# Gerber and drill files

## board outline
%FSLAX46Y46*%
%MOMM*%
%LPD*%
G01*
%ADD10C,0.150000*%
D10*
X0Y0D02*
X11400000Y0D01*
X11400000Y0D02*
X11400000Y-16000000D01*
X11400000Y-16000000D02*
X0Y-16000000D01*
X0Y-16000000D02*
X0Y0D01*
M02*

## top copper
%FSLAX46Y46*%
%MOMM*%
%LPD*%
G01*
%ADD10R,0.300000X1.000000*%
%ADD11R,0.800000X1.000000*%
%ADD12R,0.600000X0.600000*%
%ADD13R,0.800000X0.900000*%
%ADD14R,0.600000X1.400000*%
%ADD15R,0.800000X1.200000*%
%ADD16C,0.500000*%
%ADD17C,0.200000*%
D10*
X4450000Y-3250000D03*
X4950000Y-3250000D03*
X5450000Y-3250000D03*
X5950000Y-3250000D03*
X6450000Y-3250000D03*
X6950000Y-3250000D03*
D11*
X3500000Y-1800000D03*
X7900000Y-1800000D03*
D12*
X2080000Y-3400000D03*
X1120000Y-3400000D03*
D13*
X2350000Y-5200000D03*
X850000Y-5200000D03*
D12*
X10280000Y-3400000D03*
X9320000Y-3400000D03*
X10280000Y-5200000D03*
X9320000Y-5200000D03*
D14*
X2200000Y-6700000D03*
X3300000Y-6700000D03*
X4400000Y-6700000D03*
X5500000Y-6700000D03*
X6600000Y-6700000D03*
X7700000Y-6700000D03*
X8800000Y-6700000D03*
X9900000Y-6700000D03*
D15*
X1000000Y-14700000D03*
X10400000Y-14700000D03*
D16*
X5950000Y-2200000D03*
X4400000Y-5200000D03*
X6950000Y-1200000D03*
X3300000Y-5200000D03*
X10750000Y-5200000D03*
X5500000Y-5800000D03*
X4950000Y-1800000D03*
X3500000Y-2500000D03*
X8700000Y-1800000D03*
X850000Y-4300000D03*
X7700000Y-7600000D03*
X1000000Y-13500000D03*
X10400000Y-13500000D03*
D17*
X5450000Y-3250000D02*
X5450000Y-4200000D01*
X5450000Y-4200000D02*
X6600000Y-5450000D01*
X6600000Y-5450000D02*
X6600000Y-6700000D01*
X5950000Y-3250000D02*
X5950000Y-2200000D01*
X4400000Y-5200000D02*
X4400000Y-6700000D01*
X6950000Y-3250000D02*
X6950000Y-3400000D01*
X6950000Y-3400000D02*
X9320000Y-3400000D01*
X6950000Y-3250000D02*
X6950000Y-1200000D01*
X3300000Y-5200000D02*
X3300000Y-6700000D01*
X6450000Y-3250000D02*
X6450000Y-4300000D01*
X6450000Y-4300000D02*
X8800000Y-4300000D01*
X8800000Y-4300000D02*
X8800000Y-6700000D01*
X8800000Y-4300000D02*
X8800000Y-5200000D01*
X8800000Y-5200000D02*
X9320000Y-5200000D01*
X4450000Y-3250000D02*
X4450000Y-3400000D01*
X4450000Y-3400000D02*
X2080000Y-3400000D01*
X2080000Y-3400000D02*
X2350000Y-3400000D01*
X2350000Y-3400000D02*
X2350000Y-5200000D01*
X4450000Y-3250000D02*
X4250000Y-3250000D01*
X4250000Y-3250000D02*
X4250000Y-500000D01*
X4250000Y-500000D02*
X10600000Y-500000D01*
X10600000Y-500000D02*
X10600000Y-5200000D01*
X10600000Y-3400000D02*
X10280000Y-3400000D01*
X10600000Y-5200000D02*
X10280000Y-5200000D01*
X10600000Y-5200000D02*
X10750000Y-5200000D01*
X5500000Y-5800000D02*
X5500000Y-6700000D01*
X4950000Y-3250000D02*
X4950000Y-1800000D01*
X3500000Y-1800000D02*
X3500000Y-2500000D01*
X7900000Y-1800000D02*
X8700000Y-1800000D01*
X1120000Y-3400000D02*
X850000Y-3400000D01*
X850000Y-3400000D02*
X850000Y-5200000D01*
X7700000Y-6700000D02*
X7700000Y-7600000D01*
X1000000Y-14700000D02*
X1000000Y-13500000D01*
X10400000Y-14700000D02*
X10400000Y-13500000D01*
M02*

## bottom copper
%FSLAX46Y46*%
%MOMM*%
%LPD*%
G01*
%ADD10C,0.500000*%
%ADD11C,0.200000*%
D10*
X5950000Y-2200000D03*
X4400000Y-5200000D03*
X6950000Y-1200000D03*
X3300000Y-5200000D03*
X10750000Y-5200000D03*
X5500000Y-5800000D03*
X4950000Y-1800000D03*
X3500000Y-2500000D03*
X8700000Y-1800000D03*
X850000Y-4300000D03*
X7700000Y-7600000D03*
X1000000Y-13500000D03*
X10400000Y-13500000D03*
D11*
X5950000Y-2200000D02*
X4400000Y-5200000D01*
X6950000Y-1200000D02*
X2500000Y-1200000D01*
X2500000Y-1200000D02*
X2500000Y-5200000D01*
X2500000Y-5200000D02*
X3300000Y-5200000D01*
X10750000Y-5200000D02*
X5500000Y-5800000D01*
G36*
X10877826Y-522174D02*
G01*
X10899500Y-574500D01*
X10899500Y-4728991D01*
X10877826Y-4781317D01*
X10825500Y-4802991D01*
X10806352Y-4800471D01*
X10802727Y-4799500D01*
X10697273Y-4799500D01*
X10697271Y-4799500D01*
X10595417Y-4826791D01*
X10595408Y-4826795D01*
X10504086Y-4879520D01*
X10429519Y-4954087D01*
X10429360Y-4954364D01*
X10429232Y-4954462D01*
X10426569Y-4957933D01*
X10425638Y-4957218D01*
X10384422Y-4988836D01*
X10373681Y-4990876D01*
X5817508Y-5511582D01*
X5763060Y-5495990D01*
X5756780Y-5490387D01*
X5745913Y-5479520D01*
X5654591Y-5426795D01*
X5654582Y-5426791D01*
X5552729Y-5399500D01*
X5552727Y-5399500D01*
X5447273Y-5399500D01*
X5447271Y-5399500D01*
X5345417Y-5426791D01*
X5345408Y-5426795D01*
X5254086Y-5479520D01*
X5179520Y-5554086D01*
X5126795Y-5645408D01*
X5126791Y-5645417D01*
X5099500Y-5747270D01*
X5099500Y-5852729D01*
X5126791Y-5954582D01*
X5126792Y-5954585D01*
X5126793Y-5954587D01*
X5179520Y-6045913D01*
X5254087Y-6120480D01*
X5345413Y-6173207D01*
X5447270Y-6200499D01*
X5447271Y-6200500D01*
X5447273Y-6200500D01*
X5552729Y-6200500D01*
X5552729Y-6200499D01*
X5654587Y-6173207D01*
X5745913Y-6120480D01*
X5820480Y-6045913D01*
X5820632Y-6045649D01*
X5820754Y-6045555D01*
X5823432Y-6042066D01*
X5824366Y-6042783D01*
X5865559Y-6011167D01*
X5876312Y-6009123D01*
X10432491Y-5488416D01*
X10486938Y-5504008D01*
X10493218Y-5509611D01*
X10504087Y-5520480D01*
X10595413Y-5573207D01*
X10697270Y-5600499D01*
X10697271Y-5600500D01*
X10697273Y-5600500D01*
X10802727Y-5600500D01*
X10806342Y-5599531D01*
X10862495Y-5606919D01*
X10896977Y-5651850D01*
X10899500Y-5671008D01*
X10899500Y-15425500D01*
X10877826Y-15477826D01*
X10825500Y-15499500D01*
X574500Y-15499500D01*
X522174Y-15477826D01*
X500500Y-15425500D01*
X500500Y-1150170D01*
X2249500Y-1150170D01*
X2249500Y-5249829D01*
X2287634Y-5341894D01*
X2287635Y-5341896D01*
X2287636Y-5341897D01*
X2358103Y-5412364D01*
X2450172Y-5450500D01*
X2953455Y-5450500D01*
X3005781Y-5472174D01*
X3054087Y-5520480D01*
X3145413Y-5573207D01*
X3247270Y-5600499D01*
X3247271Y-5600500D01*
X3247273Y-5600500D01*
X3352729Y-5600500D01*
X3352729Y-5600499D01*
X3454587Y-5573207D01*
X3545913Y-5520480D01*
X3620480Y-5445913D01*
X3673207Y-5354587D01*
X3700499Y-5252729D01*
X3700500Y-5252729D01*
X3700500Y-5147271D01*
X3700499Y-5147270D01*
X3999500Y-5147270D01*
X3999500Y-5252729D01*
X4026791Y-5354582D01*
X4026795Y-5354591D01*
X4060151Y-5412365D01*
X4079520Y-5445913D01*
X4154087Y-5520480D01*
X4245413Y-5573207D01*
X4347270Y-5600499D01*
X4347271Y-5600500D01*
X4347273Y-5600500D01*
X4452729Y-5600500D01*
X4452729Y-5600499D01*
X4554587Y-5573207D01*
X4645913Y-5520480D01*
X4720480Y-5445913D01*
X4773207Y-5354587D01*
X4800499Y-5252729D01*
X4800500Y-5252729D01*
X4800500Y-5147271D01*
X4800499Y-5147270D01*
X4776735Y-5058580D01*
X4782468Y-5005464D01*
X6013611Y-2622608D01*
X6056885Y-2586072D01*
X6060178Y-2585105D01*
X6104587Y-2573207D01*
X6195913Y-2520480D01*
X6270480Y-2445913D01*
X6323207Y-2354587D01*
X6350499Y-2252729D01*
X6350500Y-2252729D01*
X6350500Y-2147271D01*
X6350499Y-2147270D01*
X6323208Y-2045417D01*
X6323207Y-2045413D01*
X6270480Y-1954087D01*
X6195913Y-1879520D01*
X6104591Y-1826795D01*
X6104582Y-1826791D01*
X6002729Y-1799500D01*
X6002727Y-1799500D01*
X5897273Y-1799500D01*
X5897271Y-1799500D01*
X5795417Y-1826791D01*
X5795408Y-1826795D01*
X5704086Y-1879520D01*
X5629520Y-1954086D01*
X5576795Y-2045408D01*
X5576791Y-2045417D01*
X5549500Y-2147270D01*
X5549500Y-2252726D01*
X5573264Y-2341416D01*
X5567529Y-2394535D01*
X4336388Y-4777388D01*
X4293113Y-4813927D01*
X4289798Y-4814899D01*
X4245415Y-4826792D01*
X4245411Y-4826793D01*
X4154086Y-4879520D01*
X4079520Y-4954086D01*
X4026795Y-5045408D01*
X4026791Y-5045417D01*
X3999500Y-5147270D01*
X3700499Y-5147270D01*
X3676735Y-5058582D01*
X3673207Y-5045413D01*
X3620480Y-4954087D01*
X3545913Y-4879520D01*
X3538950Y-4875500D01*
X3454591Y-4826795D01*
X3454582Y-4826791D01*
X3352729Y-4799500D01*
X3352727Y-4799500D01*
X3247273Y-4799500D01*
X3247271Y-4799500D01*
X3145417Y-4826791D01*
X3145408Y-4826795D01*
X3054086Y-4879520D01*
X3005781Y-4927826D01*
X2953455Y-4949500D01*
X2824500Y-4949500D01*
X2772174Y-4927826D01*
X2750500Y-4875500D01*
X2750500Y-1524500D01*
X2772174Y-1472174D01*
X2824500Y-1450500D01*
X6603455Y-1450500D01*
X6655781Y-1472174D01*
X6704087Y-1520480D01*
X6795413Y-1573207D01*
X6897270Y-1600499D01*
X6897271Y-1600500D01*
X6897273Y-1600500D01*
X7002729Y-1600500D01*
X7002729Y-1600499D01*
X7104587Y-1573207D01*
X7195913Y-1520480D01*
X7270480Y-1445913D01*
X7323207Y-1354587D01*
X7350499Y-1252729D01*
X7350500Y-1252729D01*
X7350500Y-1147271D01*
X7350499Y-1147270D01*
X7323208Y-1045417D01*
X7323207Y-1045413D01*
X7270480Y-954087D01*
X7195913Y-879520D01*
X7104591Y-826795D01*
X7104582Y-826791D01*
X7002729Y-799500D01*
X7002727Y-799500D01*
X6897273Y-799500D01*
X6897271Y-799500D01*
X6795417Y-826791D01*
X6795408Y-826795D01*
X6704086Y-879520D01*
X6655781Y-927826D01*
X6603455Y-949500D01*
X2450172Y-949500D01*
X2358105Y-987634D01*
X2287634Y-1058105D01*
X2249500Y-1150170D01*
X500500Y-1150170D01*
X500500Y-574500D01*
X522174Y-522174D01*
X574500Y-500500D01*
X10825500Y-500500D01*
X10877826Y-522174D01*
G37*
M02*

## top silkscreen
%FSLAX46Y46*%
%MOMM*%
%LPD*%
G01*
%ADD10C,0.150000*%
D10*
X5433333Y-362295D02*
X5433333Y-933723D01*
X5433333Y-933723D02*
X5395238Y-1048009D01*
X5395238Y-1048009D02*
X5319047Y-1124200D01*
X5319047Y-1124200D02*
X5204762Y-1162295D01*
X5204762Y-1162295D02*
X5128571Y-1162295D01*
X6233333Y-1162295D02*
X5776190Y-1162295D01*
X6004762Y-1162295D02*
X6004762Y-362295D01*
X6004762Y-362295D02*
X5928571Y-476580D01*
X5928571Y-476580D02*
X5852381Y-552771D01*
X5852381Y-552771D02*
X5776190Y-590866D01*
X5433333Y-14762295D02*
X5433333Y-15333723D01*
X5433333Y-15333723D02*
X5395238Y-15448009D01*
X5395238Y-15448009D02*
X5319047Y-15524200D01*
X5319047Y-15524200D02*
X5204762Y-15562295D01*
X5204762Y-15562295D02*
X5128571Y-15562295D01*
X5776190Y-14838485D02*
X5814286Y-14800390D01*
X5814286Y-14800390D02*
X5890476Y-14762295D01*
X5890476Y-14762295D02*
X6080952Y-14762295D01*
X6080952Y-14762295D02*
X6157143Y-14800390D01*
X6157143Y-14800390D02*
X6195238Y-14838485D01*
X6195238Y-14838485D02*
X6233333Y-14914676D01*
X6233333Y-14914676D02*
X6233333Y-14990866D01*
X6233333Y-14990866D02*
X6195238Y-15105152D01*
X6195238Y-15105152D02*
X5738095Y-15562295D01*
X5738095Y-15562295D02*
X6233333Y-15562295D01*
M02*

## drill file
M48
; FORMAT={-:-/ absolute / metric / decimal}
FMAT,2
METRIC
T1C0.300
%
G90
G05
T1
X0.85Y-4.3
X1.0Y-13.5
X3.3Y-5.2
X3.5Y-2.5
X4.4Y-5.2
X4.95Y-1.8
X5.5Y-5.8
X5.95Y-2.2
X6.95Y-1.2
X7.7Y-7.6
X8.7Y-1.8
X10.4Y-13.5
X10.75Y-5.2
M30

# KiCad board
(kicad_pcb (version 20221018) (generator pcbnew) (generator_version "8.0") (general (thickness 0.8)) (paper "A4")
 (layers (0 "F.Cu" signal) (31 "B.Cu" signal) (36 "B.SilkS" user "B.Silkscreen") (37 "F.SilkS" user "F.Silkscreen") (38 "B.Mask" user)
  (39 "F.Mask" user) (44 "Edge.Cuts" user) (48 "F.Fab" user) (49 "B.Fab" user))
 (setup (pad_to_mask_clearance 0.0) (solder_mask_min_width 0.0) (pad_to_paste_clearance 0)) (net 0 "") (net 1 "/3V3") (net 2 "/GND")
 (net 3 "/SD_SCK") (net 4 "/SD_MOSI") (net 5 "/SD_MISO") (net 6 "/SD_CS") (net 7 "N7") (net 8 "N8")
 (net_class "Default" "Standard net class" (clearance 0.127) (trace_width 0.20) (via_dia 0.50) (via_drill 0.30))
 (gr_line (start 0 0) (end 11.4 0) (layer "Edge.Cuts") (width 0.15))
 (gr_line (start 11.4 0) (end 11.4 16.0) (layer "Edge.Cuts") (width 0.15))
 (gr_line (start 11.4 16.0) (end 0 16.0) (layer "Edge.Cuts") (width 0.15))
 (gr_line (start 0 16.0) (end 0 0) (layer "Edge.Cuts") (width 0.15))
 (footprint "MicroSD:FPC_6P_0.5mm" (layer "F.Cu") (at 5.7 2.0)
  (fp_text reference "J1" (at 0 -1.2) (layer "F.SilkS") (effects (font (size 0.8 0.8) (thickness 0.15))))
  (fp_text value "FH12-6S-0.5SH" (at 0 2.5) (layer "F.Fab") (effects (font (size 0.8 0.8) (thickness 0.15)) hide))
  (pad "1" smd rect (at -1.25 1.25) (size 0.30 1.00) (layers "F.Cu" "F.Paste" "F.Mask") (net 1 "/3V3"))
  (pad "2" smd rect (at -0.75 1.25) (size 0.30 1.00) (layers "F.Cu" "F.Paste" "F.Mask") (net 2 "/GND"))
  (pad "3" smd rect (at -0.25 1.25) (size 0.30 1.00) (layers "F.Cu" "F.Paste" "F.Mask") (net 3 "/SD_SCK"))
  (pad "4" smd rect (at 0.25 1.25) (size 0.30 1.00) (layers "F.Cu" "F.Paste" "F.Mask") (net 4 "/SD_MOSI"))
  (pad "5" smd rect (at 0.75 1.25) (size 0.30 1.00) (layers "F.Cu" "F.Paste" "F.Mask") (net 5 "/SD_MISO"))
  (pad "6" smd rect (at 1.25 1.25) (size 0.30 1.00) (layers "F.Cu" "F.Paste" "F.Mask") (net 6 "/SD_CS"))
  (pad "MP1" smd rect (at -2.2 -0.2) (size 0.8 1.0) (layers "F.Cu" "F.Paste" "F.Mask") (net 2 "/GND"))
  (pad "MP2" smd rect (at 2.2 -0.2) (size 0.8 1.0) (layers "F.Cu" "F.Paste" "F.Mask") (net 2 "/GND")))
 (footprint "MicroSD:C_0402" (layer "F.Cu") (at 1.60 3.40)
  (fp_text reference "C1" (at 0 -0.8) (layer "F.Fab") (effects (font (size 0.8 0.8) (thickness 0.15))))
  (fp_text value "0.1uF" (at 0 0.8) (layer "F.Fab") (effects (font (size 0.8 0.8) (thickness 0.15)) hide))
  (pad "1" smd rect (at 0.48 0) (size 0.6 0.6) (layers "F.Cu" "F.Paste" "F.Mask") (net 1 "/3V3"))
  (pad "2" smd rect (at -0.48 0) (size 0.6 0.6) (layers "F.Cu" "F.Paste" "F.Mask") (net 2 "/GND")))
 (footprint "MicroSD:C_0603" (layer "F.Cu") (at 1.60 5.20)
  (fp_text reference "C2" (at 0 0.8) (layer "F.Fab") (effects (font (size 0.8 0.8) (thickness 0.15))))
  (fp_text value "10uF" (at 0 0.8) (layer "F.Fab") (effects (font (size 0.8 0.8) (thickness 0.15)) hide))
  (pad "1" smd rect (at 0.75 0) (size 0.8 0.9) (layers "F.Cu" "F.Paste" "F.Mask") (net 1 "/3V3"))
  (pad "2" smd rect (at -0.75 0) (size 0.8 0.9) (layers "F.Cu" "F.Paste" "F.Mask") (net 2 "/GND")))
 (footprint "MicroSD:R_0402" (layer "F.Cu") (at 9.80 3.40)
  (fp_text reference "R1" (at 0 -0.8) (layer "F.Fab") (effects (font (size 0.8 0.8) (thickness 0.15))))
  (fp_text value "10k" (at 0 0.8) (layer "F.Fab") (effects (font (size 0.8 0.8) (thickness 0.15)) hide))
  (pad "1" smd rect (at 0.48 0) (size 0.6 0.6) (layers "F.Cu" "F.Paste" "F.Mask") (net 1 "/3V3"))
  (pad "2" smd rect (at -0.48 0) (size 0.6 0.6) (layers "F.Cu" "F.Paste" "F.Mask") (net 6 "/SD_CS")))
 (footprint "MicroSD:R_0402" (layer "F.Cu") (at 9.80 5.20)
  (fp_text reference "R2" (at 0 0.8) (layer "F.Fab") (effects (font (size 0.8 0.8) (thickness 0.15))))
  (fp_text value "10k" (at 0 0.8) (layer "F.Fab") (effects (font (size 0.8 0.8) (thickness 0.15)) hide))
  (pad "1" smd rect (at 0.48 0) (size 0.6 0.6) (layers "F.Cu" "F.Paste" "F.Mask") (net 1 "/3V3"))
  (pad "2" smd rect (at -0.48 0) (size 0.6 0.6) (layers "F.Cu" "F.Paste" "F.Mask") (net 5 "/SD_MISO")))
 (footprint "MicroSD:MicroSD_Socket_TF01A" (layer "F.Cu") (at 5.70 11.20)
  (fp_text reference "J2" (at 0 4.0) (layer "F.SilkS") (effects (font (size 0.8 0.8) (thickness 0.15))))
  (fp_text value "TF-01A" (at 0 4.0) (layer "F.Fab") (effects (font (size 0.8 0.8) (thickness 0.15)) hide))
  (pad "1" smd rect (at -3.5 -4.5) (size 0.60 1.40) (layers "F.Cu" "F.Paste" "F.Mask") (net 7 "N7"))
  (pad "2" smd rect (at -2.4 -4.5) (size 0.60 1.40) (layers "F.Cu" "F.Paste" "F.Mask") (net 6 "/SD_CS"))
  (pad "3" smd rect (at -1.3 -4.5) (size 0.60 1.40) (layers "F.Cu" "F.Paste" "F.Mask") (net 4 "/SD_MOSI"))
  (pad "4" smd rect (at -0.2 -4.5) (size 0.60 1.40) (layers "F.Cu" "F.Paste" "F.Mask") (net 1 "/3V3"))
  (pad "5" smd rect (at 0.9 -4.5) (size 0.60 1.40) (layers "F.Cu" "F.Paste" "F.Mask") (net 3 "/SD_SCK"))
  (pad "6" smd rect (at 2.0 -4.5) (size 0.60 1.40) (layers "F.Cu" "F.Paste" "F.Mask") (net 2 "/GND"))
  (pad "7" smd rect (at 3.1 -4.5) (size 0.60 1.40) (layers "F.Cu" "F.Paste" "F.Mask") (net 5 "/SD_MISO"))
  (pad "8" smd rect (at 4.2 -4.5) (size 0.60 1.40) (layers "F.Cu" "F.Paste" "F.Mask") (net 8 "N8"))
  (pad "9" smd rect (at -4.7 3.5) (size 0.80 1.20) (layers "F.Cu" "F.Paste" "F.Mask") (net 2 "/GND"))
  (pad "10" smd rect (at 4.7 3.5) (size 0.80 1.20) (layers "F.Cu" "F.Paste" "F.Mask") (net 2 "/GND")))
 (segment (start 5.450 3.250) (end 5.450 4.200) (width 0.200) (layer "F.Cu") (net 3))
 (segment (start 5.450 4.200) (end 6.600 5.450) (width 0.200) (layer "F.Cu") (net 3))
 (segment (start 6.600 5.450) (end 6.600 6.700) (width 0.200) (layer "F.Cu") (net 3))
 (segment (start 5.950 3.250) (end 5.950 2.200) (width 0.200) (layer "F.Cu") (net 4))
 (segment (start 5.950 2.200) (end 4.400 5.200) (width 0.200) (layer "B.Cu") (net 4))
 (segment (start 4.400 5.200) (end 4.400 6.700) (width 0.200) (layer "F.Cu") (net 4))
 (segment (start 6.950 3.250) (end 6.950 3.400) (width 0.200) (layer "F.Cu") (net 6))
 (segment (start 6.950 3.400) (end 9.320 3.400) (width 0.200) (layer "F.Cu") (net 6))
 (segment (start 6.950 3.250) (end 6.950 1.200) (width 0.200) (layer "F.Cu") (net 6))
 (segment (start 6.950 1.200) (end 2.500 1.200) (width 0.200) (layer "B.Cu") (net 6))
 (segment (start 2.500 1.200) (end 2.500 5.200) (width 0.200) (layer "B.Cu") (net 6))
 (segment (start 2.500 5.200) (end 3.300 5.200) (width 0.200) (layer "B.Cu") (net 6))
 (segment (start 3.300 5.200) (end 3.300 6.700) (width 0.200) (layer "F.Cu") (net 6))
 (segment (start 6.450 3.250) (end 6.450 4.300) (width 0.200) (layer "F.Cu") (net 5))
 (segment (start 6.450 4.300) (end 8.800 4.300) (width 0.200) (layer "F.Cu") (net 5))
 (segment (start 8.800 4.300) (end 8.800 6.700) (width 0.200) (layer "F.Cu") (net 5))
 (segment (start 8.800 4.300) (end 8.800 5.200) (width 0.200) (layer "F.Cu") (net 5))
 (segment (start 8.800 5.200) (end 9.320 5.200) (width 0.200) (layer "F.Cu") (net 5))
 (segment (start 4.450 3.250) (end 4.450 3.400) (width 0.200) (layer "F.Cu") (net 1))
 (segment (start 4.450 3.400) (end 2.080 3.400) (width 0.200) (layer "F.Cu") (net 1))
 (segment (start 2.080 3.400) (end 2.350 3.400) (width 0.200) (layer "F.Cu") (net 1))
 (segment (start 2.350 3.400) (end 2.350 5.200) (width 0.200) (layer "F.Cu") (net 1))
 (segment (start 4.450 3.250) (end 4.250 3.250) (width 0.200) (layer "F.Cu") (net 1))
 (segment (start 4.250 3.250) (end 4.250 0.500) (width 0.200) (layer "F.Cu") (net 1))
 (segment (start 4.250 0.500) (end 10.600 0.500) (width 0.200) (layer "F.Cu") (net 1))
 (segment (start 10.600 0.500) (end 10.600 5.200) (width 0.200) (layer "F.Cu") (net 1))
 (segment (start 10.600 3.400) (end 10.280 3.400) (width 0.200) (layer "F.Cu") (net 1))
 (segment (start 10.600 5.200) (end 10.280 5.200) (width 0.200) (layer "F.Cu") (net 1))
 (segment (start 10.600 5.200) (end 10.750 5.200) (width 0.200) (layer "F.Cu") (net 1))
 (segment (start 10.750 5.200) (end 5.500 5.800) (width 0.200) (layer "B.Cu") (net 1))
 (segment (start 5.500 5.800) (end 5.500 6.700) (width 0.200) (layer "F.Cu") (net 1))
 (segment (start 4.950 3.250) (end 4.950 1.800) (width 0.200) (layer "F.Cu") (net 2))
 (segment (start 3.500 1.800) (end 3.500 2.500) (width 0.200) (layer "F.Cu") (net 2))
 (segment (start 7.900 1.800) (end 8.700 1.800) (width 0.200) (layer "F.Cu") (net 2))
 (segment (start 1.120 3.400) (end 0.850 3.400) (width 0.200) (layer "F.Cu") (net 2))
 (segment (start 0.850 3.400) (end 0.850 5.200) (width 0.200) (layer "F.Cu") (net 2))
 (segment (start 7.700 6.700) (end 7.700 7.600) (width 0.200) (layer "F.Cu") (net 2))
 (segment (start 1.000 14.700) (end 1.000 13.500) (width 0.200) (layer "F.Cu") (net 2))
 (segment (start 10.400 14.700) (end 10.400 13.500) (width 0.200) (layer "F.Cu") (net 2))
 (via (at 5.950 2.200) (size 0.500) (drill 0.300) (layers "F.Cu" "B.Cu") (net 4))
 (via (at 4.400 5.200) (size 0.500) (drill 0.300) (layers "F.Cu" "B.Cu") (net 4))
 (via (at 6.950 1.200) (size 0.500) (drill 0.300) (layers "F.Cu" "B.Cu") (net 6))
 (via (at 3.300 5.200) (size 0.500) (drill 0.300) (layers "F.Cu" "B.Cu") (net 6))
 (via (at 10.750 5.200) (size 0.500) (drill 0.300) (layers "F.Cu" "B.Cu") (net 1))
 (via (at 5.500 5.800) (size 0.500) (drill 0.300) (layers "F.Cu" "B.Cu") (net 1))
 (via (at 4.950 1.800) (size 0.500) (drill 0.300) (layers "F.Cu" "B.Cu") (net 2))
 (via (at 3.500 2.500) (size 0.500) (drill 0.300) (layers "F.Cu" "B.Cu") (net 2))
 (via (at 8.700 1.800) (size 0.500) (drill 0.300) (layers "F.Cu" "B.Cu") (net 2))
 (via (at 0.850 4.300) (size 0.500) (drill 0.300) (layers "F.Cu" "B.Cu") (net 2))
 (via (at 7.700 7.600) (size 0.500) (drill 0.300) (layers "F.Cu" "B.Cu") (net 2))
 (via (at 1.000 13.500) (size 0.500) (drill 0.300) (layers "F.Cu" "B.Cu") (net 2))
 (via (at 10.400 13.500) (size 0.500) (drill 0.300) (layers "F.Cu" "B.Cu") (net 2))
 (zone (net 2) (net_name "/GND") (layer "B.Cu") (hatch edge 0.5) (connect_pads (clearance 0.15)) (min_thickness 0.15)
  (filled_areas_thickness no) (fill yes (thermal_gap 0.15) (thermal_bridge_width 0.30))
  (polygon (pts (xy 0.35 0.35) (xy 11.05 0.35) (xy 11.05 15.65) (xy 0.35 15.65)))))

